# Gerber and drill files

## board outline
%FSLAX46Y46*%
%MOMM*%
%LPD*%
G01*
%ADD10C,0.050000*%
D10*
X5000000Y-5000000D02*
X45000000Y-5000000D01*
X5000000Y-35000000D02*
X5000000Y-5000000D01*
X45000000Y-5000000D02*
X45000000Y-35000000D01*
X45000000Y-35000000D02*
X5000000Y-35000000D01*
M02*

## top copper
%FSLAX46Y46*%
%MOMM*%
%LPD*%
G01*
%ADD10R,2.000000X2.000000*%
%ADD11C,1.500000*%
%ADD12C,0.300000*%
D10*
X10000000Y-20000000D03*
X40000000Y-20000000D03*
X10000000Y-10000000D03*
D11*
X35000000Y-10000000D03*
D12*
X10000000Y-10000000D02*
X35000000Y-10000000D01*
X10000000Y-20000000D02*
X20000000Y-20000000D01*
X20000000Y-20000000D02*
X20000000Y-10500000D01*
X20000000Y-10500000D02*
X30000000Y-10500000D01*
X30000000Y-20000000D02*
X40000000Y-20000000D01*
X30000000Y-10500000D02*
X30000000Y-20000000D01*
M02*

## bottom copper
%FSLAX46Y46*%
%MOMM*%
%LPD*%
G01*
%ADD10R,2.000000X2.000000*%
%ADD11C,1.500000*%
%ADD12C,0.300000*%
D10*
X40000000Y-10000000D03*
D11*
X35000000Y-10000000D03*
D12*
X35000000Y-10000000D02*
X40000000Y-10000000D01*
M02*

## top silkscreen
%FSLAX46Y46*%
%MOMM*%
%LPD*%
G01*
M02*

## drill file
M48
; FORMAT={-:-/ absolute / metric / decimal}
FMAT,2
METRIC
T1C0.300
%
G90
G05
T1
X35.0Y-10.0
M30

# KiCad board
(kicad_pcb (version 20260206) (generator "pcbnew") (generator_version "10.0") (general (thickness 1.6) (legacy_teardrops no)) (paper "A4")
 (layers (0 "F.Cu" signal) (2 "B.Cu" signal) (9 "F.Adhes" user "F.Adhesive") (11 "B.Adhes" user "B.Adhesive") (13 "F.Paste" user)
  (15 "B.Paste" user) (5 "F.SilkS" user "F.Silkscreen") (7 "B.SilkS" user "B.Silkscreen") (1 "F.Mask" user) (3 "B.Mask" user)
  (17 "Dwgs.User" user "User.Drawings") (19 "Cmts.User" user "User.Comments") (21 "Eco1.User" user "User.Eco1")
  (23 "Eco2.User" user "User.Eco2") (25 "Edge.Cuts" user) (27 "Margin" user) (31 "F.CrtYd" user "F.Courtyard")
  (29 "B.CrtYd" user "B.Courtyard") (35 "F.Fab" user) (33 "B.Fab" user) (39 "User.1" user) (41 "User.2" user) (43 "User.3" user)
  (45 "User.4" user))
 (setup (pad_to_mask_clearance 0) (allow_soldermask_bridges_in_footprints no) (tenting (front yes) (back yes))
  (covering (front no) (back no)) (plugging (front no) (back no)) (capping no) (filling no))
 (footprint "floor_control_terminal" (layer "F.Cu") (at 10 20)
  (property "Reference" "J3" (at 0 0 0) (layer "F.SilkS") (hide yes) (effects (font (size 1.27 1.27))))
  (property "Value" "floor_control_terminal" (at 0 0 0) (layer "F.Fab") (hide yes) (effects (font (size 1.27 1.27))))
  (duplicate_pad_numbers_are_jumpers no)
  (pad "1" smd rect (at 0 0) (size 2 2) (layers "F.Cu" "F.Mask" "F.Paste") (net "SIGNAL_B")))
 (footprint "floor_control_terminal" (layer "F.Cu") (at 40 20)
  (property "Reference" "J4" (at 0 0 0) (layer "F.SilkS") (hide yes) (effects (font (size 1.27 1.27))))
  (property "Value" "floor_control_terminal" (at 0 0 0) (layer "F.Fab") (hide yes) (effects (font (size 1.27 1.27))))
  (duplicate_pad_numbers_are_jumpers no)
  (pad "1" smd rect (at 0 0) (size 2 2) (layers "F.Cu" "F.Mask" "F.Paste") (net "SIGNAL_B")))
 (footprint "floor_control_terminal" (layer "F.Cu") (at 10 10)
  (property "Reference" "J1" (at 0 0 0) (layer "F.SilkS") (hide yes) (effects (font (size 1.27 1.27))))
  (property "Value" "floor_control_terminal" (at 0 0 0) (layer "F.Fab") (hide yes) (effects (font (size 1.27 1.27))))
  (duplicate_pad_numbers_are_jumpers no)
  (pad "1" smd rect (at 0 0) (size 2 2) (layers "F.Cu" "F.Mask" "F.Paste") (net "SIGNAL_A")))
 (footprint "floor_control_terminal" (layer "B.Cu") (at 40 10)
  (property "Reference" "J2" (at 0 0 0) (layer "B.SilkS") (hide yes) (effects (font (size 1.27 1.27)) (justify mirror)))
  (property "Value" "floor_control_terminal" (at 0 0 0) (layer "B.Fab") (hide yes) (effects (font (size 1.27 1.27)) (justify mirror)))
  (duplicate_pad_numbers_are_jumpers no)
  (pad "1" smd rect (at 0 0) (size 2 2) (layers "B.Cu" "B.Mask" "B.Paste") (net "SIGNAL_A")))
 (gr_line (start 5 5) (end 45 5) (stroke (width 0.05) (type default)) (layer "Edge.Cuts"))
 (gr_line (start 5 35) (end 5 5) (stroke (width 0.05) (type default)) (layer "Edge.Cuts"))
 (gr_line (start 45 5) (end 45 35) (stroke (width 0.05) (type default)) (layer "Edge.Cuts"))
 (gr_line (start 45 35) (end 5 35) (stroke (width 0.05) (type default)) (layer "Edge.Cuts"))
 (segment (start 10 10) (end 35 10) (width 0.3) (layer "F.Cu") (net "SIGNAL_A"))
 (via (at 35 10) (size 1.5) (drill 0.3) (layers "F.Cu" "B.Cu") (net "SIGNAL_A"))
 (segment (start 35 10) (end 40 10) (width 0.3) (layer "B.Cu") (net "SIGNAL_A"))
 (segment (start 10 20) (end 20 20) (width 0.3) (layer "F.Cu") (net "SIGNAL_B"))
 (segment (start 20 20) (end 20 10.5) (width 0.3) (layer "F.Cu") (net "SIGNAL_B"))
 (segment (start 20 10.5) (end 30 10.5) (width 0.3) (layer "F.Cu") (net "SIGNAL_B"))
 (segment (start 30 20) (end 40 20) (width 0.3) (layer "F.Cu") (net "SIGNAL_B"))
 (segment (start 30 10.5) (end 30 20) (width 0.3) (layer "F.Cu") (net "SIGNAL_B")))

